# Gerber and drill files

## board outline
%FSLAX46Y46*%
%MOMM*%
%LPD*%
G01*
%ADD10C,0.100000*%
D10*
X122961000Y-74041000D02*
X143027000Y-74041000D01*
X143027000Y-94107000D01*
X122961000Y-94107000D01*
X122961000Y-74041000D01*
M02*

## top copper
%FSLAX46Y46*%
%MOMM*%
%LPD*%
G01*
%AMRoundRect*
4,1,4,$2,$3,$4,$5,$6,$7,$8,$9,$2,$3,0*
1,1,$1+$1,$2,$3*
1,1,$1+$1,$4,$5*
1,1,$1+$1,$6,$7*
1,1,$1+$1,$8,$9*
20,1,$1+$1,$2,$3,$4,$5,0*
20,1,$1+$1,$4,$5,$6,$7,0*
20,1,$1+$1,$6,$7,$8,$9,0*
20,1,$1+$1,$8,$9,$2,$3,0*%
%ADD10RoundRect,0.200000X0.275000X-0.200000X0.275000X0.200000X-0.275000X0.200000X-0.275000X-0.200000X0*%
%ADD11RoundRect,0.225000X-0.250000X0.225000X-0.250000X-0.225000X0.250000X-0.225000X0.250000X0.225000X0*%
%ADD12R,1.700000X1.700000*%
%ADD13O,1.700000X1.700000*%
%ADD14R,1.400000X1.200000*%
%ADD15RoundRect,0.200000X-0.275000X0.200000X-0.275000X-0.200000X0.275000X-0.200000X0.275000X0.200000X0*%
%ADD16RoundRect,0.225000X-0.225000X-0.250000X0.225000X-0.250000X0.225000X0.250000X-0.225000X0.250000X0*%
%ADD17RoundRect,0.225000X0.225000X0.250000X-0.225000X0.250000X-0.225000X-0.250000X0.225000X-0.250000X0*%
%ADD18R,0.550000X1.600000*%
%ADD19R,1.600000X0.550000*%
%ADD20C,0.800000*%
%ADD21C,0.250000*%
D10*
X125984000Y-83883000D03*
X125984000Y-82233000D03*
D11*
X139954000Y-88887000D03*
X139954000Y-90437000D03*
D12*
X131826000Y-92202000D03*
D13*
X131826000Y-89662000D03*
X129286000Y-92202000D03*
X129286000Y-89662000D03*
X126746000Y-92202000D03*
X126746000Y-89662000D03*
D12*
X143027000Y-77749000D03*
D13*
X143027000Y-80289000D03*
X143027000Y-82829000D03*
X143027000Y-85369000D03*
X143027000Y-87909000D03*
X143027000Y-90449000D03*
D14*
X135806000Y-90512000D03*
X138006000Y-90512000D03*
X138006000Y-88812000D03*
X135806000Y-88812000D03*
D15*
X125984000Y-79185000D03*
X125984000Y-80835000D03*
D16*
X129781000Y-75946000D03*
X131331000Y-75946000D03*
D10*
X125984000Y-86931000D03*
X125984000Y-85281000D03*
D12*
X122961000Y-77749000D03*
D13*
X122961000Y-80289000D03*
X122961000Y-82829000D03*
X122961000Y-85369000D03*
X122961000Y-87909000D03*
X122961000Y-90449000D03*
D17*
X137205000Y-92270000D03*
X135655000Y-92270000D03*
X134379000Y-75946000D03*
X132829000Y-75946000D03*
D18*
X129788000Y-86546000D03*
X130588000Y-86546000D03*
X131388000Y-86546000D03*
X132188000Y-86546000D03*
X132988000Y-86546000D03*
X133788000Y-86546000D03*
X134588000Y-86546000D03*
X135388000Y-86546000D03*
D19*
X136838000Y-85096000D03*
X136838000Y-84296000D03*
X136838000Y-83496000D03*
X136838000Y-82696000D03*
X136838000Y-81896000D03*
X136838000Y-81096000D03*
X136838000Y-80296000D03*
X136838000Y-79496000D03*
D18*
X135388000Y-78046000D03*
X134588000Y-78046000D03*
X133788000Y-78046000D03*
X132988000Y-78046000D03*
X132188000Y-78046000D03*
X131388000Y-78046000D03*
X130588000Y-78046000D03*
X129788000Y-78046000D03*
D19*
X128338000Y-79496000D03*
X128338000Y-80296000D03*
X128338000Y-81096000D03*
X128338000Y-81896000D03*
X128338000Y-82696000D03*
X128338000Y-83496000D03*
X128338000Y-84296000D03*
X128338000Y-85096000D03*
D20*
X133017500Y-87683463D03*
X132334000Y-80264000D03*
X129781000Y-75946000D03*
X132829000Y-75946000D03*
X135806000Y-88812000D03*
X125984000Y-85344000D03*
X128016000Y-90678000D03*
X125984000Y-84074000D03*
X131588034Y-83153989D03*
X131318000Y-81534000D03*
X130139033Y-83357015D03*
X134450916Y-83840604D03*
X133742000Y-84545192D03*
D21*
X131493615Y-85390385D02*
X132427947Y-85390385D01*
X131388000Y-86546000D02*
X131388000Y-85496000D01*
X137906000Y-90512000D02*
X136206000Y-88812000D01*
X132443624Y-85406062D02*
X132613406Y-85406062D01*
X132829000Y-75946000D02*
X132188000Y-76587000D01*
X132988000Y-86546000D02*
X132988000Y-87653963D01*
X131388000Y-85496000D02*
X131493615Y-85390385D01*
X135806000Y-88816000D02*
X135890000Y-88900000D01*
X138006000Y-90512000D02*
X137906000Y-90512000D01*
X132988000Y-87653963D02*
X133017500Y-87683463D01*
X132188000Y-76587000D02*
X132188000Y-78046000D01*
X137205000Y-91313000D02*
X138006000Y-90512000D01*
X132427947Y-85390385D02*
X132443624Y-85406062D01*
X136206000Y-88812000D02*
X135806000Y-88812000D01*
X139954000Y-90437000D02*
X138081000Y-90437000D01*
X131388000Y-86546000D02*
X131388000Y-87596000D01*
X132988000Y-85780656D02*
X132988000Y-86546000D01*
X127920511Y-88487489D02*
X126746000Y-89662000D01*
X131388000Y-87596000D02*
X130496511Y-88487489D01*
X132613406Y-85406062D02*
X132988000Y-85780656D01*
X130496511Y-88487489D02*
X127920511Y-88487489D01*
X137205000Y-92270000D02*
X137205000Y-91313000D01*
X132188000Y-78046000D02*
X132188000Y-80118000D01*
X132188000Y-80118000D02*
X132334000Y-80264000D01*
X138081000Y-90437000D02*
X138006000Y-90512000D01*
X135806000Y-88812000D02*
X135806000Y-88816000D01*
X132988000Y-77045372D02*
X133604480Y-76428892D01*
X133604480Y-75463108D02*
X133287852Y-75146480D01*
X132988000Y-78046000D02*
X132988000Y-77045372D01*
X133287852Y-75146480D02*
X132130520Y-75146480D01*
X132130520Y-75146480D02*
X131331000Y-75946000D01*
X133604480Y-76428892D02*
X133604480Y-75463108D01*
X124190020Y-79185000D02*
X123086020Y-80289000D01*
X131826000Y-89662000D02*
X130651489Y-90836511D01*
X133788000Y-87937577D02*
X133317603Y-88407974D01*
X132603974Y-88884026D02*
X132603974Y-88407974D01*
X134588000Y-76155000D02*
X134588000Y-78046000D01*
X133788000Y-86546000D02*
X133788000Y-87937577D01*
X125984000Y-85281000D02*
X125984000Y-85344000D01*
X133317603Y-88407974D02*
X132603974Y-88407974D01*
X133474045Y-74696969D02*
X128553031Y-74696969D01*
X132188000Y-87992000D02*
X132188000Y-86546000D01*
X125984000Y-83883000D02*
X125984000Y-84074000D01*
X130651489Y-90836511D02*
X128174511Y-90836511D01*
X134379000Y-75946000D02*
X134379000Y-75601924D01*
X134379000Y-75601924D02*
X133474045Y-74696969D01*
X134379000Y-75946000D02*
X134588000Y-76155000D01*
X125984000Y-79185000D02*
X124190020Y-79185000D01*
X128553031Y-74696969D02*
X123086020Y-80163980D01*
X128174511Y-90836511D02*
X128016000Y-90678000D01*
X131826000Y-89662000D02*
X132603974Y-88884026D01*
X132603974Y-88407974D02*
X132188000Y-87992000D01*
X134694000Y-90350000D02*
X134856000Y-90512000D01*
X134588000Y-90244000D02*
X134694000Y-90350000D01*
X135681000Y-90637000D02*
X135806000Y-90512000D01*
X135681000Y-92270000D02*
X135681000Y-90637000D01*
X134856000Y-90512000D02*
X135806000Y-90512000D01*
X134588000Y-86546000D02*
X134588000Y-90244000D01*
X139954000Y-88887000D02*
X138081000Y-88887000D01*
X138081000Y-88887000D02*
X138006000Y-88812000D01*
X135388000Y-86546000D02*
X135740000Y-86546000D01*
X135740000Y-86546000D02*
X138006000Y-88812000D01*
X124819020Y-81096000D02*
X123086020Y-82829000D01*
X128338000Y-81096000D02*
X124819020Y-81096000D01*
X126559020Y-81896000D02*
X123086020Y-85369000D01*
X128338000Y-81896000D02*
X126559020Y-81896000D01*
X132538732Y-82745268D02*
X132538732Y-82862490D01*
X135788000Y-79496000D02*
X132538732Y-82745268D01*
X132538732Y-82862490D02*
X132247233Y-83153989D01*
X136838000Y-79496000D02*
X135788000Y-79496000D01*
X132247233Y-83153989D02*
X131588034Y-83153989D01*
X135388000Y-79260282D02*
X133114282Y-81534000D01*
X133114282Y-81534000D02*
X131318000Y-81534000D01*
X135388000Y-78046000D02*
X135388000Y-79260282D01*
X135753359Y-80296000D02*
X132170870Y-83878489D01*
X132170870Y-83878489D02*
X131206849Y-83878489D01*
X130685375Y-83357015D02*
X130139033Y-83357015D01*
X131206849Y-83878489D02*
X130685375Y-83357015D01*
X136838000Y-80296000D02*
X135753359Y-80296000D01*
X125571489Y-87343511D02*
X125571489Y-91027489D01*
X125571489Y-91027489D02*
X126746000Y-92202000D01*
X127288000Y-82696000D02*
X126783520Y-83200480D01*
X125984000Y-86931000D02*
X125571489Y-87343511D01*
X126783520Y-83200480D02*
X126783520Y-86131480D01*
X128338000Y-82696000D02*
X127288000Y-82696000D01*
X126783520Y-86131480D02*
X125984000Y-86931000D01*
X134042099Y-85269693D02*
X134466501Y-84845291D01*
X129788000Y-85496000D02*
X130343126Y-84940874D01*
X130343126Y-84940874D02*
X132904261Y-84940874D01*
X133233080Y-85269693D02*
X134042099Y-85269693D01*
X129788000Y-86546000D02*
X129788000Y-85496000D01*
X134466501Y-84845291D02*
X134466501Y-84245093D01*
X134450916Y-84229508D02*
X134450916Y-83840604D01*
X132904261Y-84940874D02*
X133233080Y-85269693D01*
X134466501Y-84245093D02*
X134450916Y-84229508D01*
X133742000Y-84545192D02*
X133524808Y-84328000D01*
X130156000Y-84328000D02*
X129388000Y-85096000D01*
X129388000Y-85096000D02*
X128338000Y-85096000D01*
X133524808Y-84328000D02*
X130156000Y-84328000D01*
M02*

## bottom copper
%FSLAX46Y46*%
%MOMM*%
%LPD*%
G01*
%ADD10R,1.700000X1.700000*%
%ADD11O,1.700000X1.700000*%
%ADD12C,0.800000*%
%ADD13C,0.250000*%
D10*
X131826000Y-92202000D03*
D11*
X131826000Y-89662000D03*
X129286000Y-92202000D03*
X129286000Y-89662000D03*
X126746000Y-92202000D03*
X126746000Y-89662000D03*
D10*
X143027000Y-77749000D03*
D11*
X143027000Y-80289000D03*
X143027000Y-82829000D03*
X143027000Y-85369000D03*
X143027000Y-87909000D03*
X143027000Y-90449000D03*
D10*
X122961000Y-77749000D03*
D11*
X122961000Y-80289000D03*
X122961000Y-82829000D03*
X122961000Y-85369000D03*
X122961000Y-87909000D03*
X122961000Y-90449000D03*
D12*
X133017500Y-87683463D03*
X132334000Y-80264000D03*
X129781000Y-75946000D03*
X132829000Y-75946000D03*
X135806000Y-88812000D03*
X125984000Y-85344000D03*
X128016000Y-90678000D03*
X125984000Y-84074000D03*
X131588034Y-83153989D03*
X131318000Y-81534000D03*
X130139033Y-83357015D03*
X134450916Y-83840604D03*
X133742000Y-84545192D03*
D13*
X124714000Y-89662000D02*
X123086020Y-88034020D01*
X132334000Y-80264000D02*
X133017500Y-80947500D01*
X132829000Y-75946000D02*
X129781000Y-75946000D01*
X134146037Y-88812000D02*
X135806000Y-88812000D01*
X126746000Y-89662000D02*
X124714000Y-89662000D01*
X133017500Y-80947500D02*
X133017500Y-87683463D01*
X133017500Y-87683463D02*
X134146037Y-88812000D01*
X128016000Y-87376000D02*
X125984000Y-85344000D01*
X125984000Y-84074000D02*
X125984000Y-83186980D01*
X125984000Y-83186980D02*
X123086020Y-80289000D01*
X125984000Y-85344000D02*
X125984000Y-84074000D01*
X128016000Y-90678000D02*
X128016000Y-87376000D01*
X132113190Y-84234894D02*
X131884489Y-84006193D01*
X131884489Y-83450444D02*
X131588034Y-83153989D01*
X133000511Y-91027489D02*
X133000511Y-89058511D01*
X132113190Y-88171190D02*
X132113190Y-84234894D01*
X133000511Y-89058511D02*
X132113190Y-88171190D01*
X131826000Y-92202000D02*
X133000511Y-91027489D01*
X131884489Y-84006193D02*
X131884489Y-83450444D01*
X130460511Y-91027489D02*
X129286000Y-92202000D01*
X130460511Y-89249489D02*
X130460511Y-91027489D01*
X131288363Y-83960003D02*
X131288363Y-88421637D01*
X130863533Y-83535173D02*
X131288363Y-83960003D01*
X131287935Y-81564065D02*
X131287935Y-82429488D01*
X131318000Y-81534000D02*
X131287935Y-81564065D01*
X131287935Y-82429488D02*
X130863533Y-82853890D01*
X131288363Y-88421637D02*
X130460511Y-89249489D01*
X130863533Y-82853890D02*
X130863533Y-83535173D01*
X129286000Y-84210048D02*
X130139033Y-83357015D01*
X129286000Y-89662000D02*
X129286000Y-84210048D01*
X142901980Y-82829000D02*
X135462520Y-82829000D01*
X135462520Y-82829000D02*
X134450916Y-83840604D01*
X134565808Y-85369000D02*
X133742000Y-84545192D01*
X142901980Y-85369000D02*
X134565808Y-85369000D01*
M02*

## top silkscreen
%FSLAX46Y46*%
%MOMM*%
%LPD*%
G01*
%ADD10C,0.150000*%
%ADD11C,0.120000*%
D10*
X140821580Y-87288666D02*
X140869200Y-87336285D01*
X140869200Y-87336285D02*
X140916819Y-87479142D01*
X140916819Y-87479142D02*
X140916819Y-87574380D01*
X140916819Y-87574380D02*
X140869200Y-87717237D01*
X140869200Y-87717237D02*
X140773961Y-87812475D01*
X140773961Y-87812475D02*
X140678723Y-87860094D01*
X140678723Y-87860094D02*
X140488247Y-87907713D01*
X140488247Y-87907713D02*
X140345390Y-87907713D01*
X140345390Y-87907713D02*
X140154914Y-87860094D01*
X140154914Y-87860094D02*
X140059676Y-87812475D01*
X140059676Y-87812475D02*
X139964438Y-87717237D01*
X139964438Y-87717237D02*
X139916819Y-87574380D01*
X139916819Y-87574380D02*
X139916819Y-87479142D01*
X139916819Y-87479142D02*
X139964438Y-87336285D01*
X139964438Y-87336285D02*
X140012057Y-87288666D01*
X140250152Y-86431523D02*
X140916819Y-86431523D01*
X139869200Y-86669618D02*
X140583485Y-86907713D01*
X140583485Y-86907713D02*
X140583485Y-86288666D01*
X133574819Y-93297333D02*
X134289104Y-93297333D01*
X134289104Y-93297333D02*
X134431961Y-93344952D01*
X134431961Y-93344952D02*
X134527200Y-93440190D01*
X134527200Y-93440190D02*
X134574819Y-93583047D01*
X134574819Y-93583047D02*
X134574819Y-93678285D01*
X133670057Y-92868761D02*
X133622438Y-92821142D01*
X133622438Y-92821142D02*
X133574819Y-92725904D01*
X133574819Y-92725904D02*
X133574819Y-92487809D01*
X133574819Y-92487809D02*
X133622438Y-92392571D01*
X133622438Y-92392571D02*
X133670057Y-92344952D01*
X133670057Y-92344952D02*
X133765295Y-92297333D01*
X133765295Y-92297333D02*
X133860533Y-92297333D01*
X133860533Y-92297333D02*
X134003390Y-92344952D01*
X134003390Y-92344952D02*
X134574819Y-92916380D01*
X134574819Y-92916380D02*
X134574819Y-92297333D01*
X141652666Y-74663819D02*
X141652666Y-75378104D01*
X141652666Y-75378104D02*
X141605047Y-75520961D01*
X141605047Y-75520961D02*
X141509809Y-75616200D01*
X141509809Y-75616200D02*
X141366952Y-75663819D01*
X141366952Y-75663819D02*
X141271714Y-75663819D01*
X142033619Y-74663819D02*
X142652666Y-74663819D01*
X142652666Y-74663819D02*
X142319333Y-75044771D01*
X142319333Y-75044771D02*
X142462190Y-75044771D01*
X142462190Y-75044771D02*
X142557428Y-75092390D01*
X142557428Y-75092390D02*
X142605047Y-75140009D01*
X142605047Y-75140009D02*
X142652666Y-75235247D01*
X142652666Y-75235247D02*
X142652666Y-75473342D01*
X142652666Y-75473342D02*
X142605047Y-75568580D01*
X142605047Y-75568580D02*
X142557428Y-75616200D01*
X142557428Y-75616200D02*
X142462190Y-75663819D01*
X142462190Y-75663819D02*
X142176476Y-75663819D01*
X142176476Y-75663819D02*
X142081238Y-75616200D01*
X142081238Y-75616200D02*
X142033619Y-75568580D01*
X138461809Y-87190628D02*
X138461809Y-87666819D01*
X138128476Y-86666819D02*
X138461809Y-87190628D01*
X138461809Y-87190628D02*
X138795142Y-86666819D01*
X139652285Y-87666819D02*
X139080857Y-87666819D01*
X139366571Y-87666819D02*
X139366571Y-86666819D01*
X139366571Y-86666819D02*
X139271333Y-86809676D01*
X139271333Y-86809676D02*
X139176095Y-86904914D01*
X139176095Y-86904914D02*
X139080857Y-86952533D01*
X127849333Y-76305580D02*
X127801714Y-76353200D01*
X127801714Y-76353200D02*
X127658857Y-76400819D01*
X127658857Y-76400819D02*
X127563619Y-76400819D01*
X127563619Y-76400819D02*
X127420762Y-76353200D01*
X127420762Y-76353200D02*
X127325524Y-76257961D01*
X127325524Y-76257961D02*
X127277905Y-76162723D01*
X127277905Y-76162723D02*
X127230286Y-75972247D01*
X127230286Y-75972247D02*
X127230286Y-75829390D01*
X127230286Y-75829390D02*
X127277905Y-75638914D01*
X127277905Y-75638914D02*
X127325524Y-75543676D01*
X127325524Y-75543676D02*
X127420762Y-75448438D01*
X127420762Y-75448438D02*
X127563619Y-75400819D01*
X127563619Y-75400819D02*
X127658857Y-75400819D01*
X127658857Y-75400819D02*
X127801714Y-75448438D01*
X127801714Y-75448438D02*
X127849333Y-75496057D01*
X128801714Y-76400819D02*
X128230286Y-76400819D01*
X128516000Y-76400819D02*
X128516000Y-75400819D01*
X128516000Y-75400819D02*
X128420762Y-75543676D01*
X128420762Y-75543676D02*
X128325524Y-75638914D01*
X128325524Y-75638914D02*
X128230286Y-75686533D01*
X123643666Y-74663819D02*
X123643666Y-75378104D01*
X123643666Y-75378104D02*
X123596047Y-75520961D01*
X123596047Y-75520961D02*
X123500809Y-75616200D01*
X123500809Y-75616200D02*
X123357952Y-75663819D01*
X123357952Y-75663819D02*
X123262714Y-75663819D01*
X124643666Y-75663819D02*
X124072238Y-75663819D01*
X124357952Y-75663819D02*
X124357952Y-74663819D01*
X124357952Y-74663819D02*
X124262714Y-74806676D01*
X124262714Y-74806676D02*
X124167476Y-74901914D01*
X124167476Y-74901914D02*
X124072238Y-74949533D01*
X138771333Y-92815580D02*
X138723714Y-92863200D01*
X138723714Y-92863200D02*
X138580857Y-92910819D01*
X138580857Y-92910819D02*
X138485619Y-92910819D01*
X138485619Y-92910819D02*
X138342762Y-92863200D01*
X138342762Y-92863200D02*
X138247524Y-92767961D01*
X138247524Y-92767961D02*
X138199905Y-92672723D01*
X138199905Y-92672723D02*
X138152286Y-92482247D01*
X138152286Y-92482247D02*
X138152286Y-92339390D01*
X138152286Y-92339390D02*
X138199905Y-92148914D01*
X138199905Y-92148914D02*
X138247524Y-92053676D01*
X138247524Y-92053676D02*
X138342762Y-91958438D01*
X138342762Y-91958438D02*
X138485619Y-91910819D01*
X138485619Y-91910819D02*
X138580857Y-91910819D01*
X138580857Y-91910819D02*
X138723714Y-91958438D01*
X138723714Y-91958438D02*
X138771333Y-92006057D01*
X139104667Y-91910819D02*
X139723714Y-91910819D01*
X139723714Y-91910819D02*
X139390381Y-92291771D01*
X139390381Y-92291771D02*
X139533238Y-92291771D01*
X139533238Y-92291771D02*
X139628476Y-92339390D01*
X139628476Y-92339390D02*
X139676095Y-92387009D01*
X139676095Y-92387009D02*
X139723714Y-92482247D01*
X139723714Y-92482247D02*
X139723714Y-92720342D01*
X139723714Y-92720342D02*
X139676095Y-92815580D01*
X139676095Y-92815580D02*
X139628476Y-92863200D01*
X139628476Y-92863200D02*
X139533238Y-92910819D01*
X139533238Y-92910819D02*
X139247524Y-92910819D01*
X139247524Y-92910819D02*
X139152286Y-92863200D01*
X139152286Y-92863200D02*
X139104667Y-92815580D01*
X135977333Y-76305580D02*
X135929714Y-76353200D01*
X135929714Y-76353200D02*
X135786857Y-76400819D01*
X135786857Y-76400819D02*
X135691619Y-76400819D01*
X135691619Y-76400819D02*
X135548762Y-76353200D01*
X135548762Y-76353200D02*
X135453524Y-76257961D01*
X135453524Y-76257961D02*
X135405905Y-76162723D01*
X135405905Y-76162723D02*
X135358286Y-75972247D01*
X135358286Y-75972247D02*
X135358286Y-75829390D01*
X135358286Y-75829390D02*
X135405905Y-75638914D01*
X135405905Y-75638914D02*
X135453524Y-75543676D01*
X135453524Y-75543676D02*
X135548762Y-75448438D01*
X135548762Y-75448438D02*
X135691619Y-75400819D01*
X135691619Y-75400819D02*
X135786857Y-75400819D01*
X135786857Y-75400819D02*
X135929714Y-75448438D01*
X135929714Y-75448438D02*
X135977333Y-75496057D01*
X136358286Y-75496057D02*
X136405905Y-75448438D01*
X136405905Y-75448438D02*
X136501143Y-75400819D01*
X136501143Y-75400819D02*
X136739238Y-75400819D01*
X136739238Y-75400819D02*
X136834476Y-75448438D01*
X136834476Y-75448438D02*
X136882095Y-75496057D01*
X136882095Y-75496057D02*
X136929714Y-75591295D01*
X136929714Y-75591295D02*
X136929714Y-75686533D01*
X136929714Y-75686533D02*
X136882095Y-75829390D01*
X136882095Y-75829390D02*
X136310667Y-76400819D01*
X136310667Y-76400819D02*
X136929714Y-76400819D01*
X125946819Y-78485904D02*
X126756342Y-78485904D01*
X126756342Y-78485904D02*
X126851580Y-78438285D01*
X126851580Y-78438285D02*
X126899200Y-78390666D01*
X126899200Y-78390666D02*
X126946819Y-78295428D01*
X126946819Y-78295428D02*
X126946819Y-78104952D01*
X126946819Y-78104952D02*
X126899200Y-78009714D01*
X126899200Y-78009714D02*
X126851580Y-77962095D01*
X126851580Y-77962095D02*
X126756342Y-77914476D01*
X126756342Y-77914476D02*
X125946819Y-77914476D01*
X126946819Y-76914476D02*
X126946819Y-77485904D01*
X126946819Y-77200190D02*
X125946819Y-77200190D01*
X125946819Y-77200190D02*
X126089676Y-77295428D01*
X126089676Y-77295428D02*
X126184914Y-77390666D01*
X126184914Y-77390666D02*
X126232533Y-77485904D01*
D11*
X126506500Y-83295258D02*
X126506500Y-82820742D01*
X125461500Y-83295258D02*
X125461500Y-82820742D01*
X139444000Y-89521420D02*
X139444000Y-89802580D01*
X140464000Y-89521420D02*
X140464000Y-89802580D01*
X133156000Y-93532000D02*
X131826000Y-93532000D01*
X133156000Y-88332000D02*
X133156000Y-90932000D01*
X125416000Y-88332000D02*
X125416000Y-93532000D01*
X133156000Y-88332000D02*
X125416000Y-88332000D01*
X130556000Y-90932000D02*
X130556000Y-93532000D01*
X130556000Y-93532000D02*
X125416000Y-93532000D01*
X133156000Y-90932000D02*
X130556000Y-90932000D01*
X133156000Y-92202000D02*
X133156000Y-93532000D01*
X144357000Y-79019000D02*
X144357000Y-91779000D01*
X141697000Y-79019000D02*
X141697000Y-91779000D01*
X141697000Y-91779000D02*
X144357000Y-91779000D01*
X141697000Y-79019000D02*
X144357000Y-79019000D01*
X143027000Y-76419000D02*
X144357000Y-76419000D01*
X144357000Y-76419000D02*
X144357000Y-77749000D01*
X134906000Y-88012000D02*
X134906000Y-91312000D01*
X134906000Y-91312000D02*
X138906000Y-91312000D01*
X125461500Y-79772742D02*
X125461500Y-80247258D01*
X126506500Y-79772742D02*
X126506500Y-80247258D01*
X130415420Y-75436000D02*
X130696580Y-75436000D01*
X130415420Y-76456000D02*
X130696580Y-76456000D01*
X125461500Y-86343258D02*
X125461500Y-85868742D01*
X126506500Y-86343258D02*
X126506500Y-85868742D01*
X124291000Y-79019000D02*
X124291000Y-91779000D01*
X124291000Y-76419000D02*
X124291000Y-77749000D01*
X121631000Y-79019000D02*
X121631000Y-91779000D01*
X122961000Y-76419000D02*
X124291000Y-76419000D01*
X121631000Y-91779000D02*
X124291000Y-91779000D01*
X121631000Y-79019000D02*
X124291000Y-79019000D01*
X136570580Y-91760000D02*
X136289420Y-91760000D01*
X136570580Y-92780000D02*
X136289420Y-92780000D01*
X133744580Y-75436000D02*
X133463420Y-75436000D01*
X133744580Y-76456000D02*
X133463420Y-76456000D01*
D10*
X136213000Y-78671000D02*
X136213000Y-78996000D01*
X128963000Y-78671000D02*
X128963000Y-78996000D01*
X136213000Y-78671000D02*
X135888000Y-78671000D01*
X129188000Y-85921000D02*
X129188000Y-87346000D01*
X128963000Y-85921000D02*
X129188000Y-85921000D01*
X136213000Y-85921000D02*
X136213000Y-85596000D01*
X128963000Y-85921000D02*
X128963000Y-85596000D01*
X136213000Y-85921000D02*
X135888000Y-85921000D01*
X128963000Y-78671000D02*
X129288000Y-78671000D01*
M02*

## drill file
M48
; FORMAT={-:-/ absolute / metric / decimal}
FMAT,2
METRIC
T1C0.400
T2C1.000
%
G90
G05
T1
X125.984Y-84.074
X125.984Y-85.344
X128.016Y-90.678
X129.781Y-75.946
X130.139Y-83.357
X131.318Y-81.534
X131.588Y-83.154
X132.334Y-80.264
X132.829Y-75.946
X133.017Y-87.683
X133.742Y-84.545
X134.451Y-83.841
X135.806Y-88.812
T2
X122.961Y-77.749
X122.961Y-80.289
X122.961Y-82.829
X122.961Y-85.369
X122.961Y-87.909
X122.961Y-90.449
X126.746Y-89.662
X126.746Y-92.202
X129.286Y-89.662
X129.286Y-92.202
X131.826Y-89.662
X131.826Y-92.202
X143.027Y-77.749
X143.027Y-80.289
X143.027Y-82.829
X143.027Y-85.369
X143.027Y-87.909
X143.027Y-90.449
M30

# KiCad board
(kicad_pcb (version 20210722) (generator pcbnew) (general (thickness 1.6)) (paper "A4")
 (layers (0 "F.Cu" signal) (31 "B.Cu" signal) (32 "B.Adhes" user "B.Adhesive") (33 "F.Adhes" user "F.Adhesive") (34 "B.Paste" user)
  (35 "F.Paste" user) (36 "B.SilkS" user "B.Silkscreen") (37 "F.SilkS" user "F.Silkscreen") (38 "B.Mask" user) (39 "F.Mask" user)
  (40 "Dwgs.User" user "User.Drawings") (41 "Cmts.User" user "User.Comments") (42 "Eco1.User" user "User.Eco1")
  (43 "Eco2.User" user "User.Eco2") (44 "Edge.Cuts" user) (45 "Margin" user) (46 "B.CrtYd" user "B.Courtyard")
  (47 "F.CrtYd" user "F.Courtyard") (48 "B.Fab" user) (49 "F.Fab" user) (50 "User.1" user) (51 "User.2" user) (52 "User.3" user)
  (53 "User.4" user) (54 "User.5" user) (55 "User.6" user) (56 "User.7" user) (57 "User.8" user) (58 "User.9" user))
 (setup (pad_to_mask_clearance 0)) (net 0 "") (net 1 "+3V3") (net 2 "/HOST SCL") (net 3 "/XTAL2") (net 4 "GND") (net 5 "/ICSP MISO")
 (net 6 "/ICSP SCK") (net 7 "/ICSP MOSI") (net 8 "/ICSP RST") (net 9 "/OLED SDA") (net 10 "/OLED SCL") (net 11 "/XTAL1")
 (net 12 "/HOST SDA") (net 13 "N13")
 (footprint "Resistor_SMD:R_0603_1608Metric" (layer "F.Cu") (at 125.984 83.058 90)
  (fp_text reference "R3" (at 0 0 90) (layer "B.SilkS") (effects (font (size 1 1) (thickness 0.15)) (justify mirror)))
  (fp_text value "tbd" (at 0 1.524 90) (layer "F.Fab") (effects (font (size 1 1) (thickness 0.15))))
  (fp_line (start -0.237258 0.5225) (end 0.237258 0.5225) (layer "F.SilkS") (width 0.12))
  (fp_line (start -0.237258 -0.5225) (end 0.237258 -0.5225) (layer "F.SilkS") (width 0.12))
  (pad "1" smd roundrect locked (at -0.825 0 90) (size 0.8 0.95) (layers "F.Cu" "F.Paste" "F.Mask") (roundrect_rratio 0.25) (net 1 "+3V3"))
  (pad "2" smd roundrect locked (at 0.825 0 90) (size 0.8 0.95) (layers "F.Cu" "F.Paste" "F.Mask") (roundrect_rratio 0.25)
   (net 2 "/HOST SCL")))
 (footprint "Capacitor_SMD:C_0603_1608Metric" (layer "F.Cu") (at 139.954 89.662 -90)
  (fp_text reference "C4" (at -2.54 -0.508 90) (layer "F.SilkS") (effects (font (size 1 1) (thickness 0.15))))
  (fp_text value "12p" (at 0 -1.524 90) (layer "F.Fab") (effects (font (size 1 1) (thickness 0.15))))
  (fp_line (start -0.14058 0.51) (end 0.14058 0.51) (layer "F.SilkS") (width 0.12))
  (fp_line (start -0.14058 -0.51) (end 0.14058 -0.51) (layer "F.SilkS") (width 0.12))
  (pad "1" smd roundrect locked (at -0.775 0 270) (size 0.9 0.95) (layers "F.Cu" "F.Paste" "F.Mask") (roundrect_rratio 0.25)
   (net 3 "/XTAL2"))
  (pad "2" smd roundrect locked (at 0.775 0 270) (size 0.9 0.95) (layers "F.Cu" "F.Paste" "F.Mask") (roundrect_rratio 0.25) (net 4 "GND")))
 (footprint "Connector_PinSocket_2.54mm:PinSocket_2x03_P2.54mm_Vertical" (layer "F.Cu") (at 131.826 92.202 -90)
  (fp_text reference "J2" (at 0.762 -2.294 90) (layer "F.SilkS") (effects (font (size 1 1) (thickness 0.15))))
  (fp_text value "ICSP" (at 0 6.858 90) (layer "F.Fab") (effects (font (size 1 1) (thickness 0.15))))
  (fp_line (start 1.33 -1.33) (end 1.33 0) (layer "F.SilkS") (width 0.12))
  (fp_line (start -3.87 -1.33) (end -1.27 -1.33) (layer "F.SilkS") (width 0.12))
  (fp_line (start -3.87 6.41) (end 1.33 6.41) (layer "F.SilkS") (width 0.12))
  (fp_line (start -3.87 -1.33) (end -3.87 6.41) (layer "F.SilkS") (width 0.12))
  (fp_line (start -1.27 1.27) (end 1.33 1.27) (layer "F.SilkS") (width 0.12))
  (fp_line (start 1.33 1.27) (end 1.33 6.41) (layer "F.SilkS") (width 0.12))
  (fp_line (start -1.27 -1.33) (end -1.27 1.27) (layer "F.SilkS") (width 0.12))
  (fp_line (start 0 -1.33) (end 1.33 -1.33) (layer "F.SilkS") (width 0.12))
  (pad "1" thru_hole rect locked (at 0 0 270) (size 1.7 1.7) (drill 1) (layers *.Cu *.Mask) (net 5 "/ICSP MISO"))
  (pad "2" thru_hole oval locked (at -2.54 0 270) (size 1.7 1.7) (drill 1) (layers *.Cu *.Mask) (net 1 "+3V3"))
  (pad "3" thru_hole oval locked (at 0 2.54 270) (size 1.7 1.7) (drill 1) (layers *.Cu *.Mask) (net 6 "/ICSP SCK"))
  (pad "4" thru_hole oval locked (at -2.54 2.54 270) (size 1.7 1.7) (drill 1) (layers *.Cu *.Mask) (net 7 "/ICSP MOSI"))
  (pad "5" thru_hole oval locked (at 0 5.08 270) (size 1.7 1.7) (drill 1) (layers *.Cu *.Mask) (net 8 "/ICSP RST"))
  (pad "6" thru_hole oval locked (at -2.54 5.08 270) (size 1.7 1.7) (drill 1) (layers *.Cu *.Mask) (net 4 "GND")))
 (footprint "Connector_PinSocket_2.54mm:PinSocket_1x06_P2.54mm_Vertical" (layer "F.Cu") (at 143.027 77.749)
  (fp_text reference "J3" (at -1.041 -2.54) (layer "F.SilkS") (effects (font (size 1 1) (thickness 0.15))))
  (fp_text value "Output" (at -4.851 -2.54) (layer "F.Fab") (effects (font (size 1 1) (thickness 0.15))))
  (fp_line (start 1.33 1.27) (end 1.33 14.03) (layer "F.SilkS") (width 0.12))
  (fp_line (start -1.33 1.27) (end -1.33 14.03) (layer "F.SilkS") (width 0.12))
  (fp_line (start -1.33 14.03) (end 1.33 14.03) (layer "F.SilkS") (width 0.12))
  (fp_line (start -1.33 1.27) (end 1.33 1.27) (layer "F.SilkS") (width 0.12))
  (fp_line (start 0 -1.33) (end 1.33 -1.33) (layer "F.SilkS") (width 0.12))
  (fp_line (start 1.33 -1.33) (end 1.33 0) (layer "F.SilkS") (width 0.12))
  (pad "1" thru_hole rect locked (at 0 0) (size 1.7 1.7) (drill 1) (layers *.Cu *.Mask))
  (pad "2" thru_hole oval locked (at 0 2.54) (size 1.7 1.7) (drill 1) (layers *.Cu *.Mask))
  (pad "3" thru_hole oval locked (at 0 5.08) (size 1.7 1.7) (drill 1) (layers *.Cu *.Mask) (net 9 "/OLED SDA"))
  (pad "4" thru_hole oval locked (at 0 7.62) (size 1.7 1.7) (drill 1) (layers *.Cu *.Mask) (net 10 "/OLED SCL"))
  (pad "5" thru_hole oval locked (at 0 10.16) (size 1.7 1.7) (drill 1) (layers *.Cu *.Mask))
  (pad "6" thru_hole oval locked (at 0 12.7) (size 1.7 1.7) (drill 1) (layers *.Cu *.Mask)))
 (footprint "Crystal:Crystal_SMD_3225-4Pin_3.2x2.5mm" (layer "F.Cu") (at 136.906 89.662)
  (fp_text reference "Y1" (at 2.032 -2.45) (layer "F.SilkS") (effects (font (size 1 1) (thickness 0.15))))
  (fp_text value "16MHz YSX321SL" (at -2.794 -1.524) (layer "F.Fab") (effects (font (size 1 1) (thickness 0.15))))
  (fp_line (start -2 -1.65) (end -2 1.65) (layer "F.SilkS") (width 0.12))
  (fp_line (start -2 1.65) (end 2 1.65) (layer "F.SilkS") (width 0.12))
  (pad "1" smd rect locked (at -1.1 0.85) (size 1.4 1.2) (layers "F.Cu" "F.Paste" "F.Mask") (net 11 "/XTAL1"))
  (pad "2" smd rect locked (at 1.1 0.85) (size 1.4 1.2) (layers "F.Cu" "F.Paste" "F.Mask") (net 4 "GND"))
  (pad "3" smd rect locked (at 1.1 -0.85) (size 1.4 1.2) (layers "F.Cu" "F.Paste" "F.Mask") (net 3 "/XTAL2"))
  (pad "4" smd rect locked (at -1.1 -0.85) (size 1.4 1.2) (layers "F.Cu" "F.Paste" "F.Mask") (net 4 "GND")))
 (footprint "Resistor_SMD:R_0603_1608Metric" (layer "F.Cu") (at 125.984 80.01 -90)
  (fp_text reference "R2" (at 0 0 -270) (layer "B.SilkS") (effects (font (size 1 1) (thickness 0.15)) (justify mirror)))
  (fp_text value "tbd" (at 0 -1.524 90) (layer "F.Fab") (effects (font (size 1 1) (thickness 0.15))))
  (fp_line (start -0.237258 0.5225) (end 0.237258 0.5225) (layer "F.SilkS") (width 0.12))
  (fp_line (start -0.237258 -0.5225) (end 0.237258 -0.5225) (layer "F.SilkS") (width 0.12))
  (pad "1" smd roundrect locked (at -0.825 0 270) (size 0.8 0.95) (layers "F.Cu" "F.Paste" "F.Mask") (roundrect_rratio 0.25) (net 1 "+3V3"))
  (pad "2" smd roundrect locked (at 0.825 0 270) (size 0.8 0.95) (layers "F.Cu" "F.Paste" "F.Mask") (roundrect_rratio 0.25)
   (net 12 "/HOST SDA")))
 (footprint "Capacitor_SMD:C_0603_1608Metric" (layer "F.Cu") (at 130.556 75.946)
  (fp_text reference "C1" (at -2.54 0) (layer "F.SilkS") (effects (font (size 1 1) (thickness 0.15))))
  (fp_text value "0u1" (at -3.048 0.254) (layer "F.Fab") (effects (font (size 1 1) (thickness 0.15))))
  (fp_line (start -0.14058 -0.51) (end 0.14058 -0.51) (layer "F.SilkS") (width 0.12))
  (fp_line (start -0.14058 0.51) (end 0.14058 0.51) (layer "F.SilkS") (width 0.12))
  (pad "1" smd roundrect locked (at -0.775 0) (size 0.9 0.95) (layers "F.Cu" "F.Paste" "F.Mask") (roundrect_rratio 0.25) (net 4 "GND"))
  (pad "2" smd roundrect locked (at 0.775 0) (size 0.9 0.95) (layers "F.Cu" "F.Paste" "F.Mask") (roundrect_rratio 0.25) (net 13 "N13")))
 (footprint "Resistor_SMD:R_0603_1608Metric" (layer "F.Cu") (at 125.984 86.106 90)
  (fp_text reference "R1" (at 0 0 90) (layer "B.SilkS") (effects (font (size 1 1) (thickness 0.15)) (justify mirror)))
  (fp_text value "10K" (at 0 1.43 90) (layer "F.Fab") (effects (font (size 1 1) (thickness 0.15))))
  (fp_line (start -0.237258 -0.5225) (end 0.237258 -0.5225) (layer "F.SilkS") (width 0.12))
  (fp_line (start -0.237258 0.5225) (end 0.237258 0.5225) (layer "F.SilkS") (width 0.12))
  (pad "1" smd roundrect locked (at -0.825 0 90) (size 0.8 0.95) (layers "F.Cu" "F.Paste" "F.Mask") (roundrect_rratio 0.25)
   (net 8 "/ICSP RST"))
  (pad "2" smd roundrect locked (at 0.825 0 90) (size 0.8 0.95) (layers "F.Cu" "F.Paste" "F.Mask") (roundrect_rratio 0.25) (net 1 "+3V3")))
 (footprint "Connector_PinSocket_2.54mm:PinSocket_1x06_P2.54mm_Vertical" (layer "F.Cu") (at 122.961 77.749)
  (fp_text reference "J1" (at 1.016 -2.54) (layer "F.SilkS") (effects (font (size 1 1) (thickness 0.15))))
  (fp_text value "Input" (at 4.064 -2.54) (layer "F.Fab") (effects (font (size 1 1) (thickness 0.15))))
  (fp_line (start 1.33 1.27) (end 1.33 14.03) (layer "F.SilkS") (width 0.12))
  (fp_line (start 1.33 -1.33) (end 1.33 0) (layer "F.SilkS") (width 0.12))
  (fp_line (start -1.33 1.27) (end -1.33 14.03) (layer "F.SilkS") (width 0.12))
  (fp_line (start 0 -1.33) (end 1.33 -1.33) (layer "F.SilkS") (width 0.12))
  (fp_line (start -1.33 14.03) (end 1.33 14.03) (layer "F.SilkS") (width 0.12))
  (fp_line (start -1.33 1.27) (end 1.33 1.27) (layer "F.SilkS") (width 0.12))
  (pad "1" thru_hole rect locked (at 0 0) (size 1.7 1.7) (drill 1) (layers *.Cu *.Mask))
  (pad "2" thru_hole oval locked (at 0 2.54) (size 1.7 1.7) (drill 1) (layers *.Cu *.Mask) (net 1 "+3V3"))
  (pad "3" thru_hole oval locked (at 0 5.08) (size 1.7 1.7) (drill 1) (layers *.Cu *.Mask) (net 12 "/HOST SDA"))
  (pad "4" thru_hole oval locked (at 0 7.62) (size 1.7 1.7) (drill 1) (layers *.Cu *.Mask) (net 2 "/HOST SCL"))
  (pad "5" thru_hole oval locked (at 0 10.16) (size 1.7 1.7) (drill 1) (layers *.Cu *.Mask) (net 4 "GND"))
  (pad "6" thru_hole oval locked (at 0 12.7) (size 1.7 1.7) (drill 1) (layers *.Cu *.Mask)))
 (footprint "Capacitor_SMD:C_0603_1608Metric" (layer "F.Cu") (at 136.43 92.27 180)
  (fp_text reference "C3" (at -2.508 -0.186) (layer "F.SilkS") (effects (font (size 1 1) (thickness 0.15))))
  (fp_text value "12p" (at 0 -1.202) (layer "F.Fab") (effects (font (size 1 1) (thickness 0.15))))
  (fp_line (start -0.14058 0.51) (end 0.14058 0.51) (layer "F.SilkS") (width 0.12))
  (fp_line (start -0.14058 -0.51) (end 0.14058 -0.51) (layer "F.SilkS") (width 0.12))
  (pad "1" smd roundrect locked (at -0.775 0 180) (size 0.9 0.95) (layers "F.Cu" "F.Paste" "F.Mask") (roundrect_rratio 0.25) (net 4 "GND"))
  (pad "2" smd roundrect locked (at 0.775 0 180) (size 0.9 0.95) (layers "F.Cu" "F.Paste" "F.Mask") (roundrect_rratio 0.25)
   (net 11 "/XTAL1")))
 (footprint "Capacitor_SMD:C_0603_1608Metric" (layer "F.Cu") (at 133.604 75.946 180)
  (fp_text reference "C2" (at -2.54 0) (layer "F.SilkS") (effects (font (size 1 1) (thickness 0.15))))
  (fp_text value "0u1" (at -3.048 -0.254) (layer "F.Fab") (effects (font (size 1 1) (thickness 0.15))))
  (fp_line (start -0.14058 0.51) (end 0.14058 0.51) (layer "F.SilkS") (width 0.12))
  (fp_line (start -0.14058 -0.51) (end 0.14058 -0.51) (layer "F.SilkS") (width 0.12))
  (pad "1" smd roundrect locked (at -0.775 0 180) (size 0.9 0.95) (layers "F.Cu" "F.Paste" "F.Mask") (roundrect_rratio 0.25) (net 1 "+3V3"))
  (pad "2" smd roundrect locked (at 0.775 0 180) (size 0.9 0.95) (layers "F.Cu" "F.Paste" "F.Mask") (roundrect_rratio 0.25) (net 4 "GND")))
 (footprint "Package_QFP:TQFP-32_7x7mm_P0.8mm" (layer "F.Cu") (at 132.588 82.296 90)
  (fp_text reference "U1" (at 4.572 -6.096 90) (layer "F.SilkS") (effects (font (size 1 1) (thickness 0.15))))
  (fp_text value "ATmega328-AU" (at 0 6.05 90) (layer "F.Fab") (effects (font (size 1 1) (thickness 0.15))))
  (fp_line (start 3.625 3.625) (end 3.3 3.625) (layer "F.SilkS") (width 0.15))
  (fp_line (start 3.625 -3.625) (end 3.3 -3.625) (layer "F.SilkS") (width 0.15))
  (fp_line (start 3.625 3.625) (end 3.625 3.3) (layer "F.SilkS") (width 0.15))
  (fp_line (start -3.625 -3.4) (end -5.05 -3.4) (layer "F.SilkS") (width 0.15))
  (fp_line (start -3.625 -3.625) (end -3.625 -3.4) (layer "F.SilkS") (width 0.15))
  (fp_line (start -3.625 3.625) (end -3.3 3.625) (layer "F.SilkS") (width 0.15))
  (fp_line (start -3.625 -3.625) (end -3.3 -3.625) (layer "F.SilkS") (width 0.15))
  (fp_line (start -3.625 3.625) (end -3.625 3.3) (layer "F.SilkS") (width 0.15))
  (fp_line (start 3.625 -3.625) (end 3.625 -3.3) (layer "F.SilkS") (width 0.15))
  (pad "1" smd rect locked (at -4.25 -2.8 90) (size 1.6 0.55) (layers "F.Cu" "F.Paste" "F.Mask") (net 9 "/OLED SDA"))
  (pad "2" smd rect locked (at -4.25 -2 90) (size 1.6 0.55) (layers "F.Cu" "F.Paste" "F.Mask"))
  (pad "3" smd rect locked (at -4.25 -1.2 90) (size 1.6 0.55) (layers "F.Cu" "F.Paste" "F.Mask") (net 4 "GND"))
  (pad "4" smd rect locked (at -4.25 -0.4 90) (size 1.6 0.55) (layers "F.Cu" "F.Paste" "F.Mask") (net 1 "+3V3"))
  (pad "5" smd rect locked (at -4.25 0.4 90) (size 1.6 0.55) (layers "F.Cu" "F.Paste" "F.Mask") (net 4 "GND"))
  (pad "6" smd rect locked (at -4.25 1.2 90) (size 1.6 0.55) (layers "F.Cu" "F.Paste" "F.Mask") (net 1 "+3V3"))
  (pad "7" smd rect locked (at -4.25 2 90) (size 1.6 0.55) (layers "F.Cu" "F.Paste" "F.Mask") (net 11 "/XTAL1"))
  (pad "8" smd rect locked (at -4.25 2.8 90) (size 1.6 0.55) (layers "F.Cu" "F.Paste" "F.Mask") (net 3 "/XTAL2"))
  (pad "9" smd rect locked (at -2.8 4.25 180) (size 1.6 0.55) (layers "F.Cu" "F.Paste" "F.Mask"))
  (pad "10" smd rect locked (at -2 4.25 180) (size 1.6 0.55) (layers "F.Cu" "F.Paste" "F.Mask"))
  (pad "11" smd rect locked (at -1.2 4.25 180) (size 1.6 0.55) (layers "F.Cu" "F.Paste" "F.Mask"))
  (pad "12" smd rect locked (at -0.4 4.25 180) (size 1.6 0.55) (layers "F.Cu" "F.Paste" "F.Mask"))
  (pad "13" smd rect locked (at 0.4 4.25 180) (size 1.6 0.55) (layers "F.Cu" "F.Paste" "F.Mask"))
  (pad "14" smd rect locked (at 1.2 4.25 180) (size 1.6 0.55) (layers "F.Cu" "F.Paste" "F.Mask"))
  (pad "15" smd rect locked (at 2 4.25 180) (size 1.6 0.55) (layers "F.Cu" "F.Paste" "F.Mask") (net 7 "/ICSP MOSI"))
  (pad "16" smd rect locked (at 2.8 4.25 180) (size 1.6 0.55) (layers "F.Cu" "F.Paste" "F.Mask") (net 5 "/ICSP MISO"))
  (pad "17" smd rect locked (at 4.25 2.8 90) (size 1.6 0.55) (layers "F.Cu" "F.Paste" "F.Mask") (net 6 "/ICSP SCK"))
  (pad "18" smd rect locked (at 4.25 2 90) (size 1.6 0.55) (layers "F.Cu" "F.Paste" "F.Mask") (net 1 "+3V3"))
  (pad "19" smd rect locked (at 4.25 1.2 90) (size 1.6 0.55) (layers "F.Cu" "F.Paste" "F.Mask"))
  (pad "20" smd rect locked (at 4.25 0.4 90) (size 1.6 0.55) (layers "F.Cu" "F.Paste" "F.Mask") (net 13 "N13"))
  (pad "21" smd rect locked (at 4.25 -0.4 90) (size 1.6 0.55) (layers "F.Cu" "F.Paste" "F.Mask") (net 4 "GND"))
  (pad "22" smd rect locked (at 4.25 -1.2 90) (size 1.6 0.55) (layers "F.Cu" "F.Paste" "F.Mask"))
  (pad "23" smd rect locked (at 4.25 -2 90) (size 1.6 0.55) (layers "F.Cu" "F.Paste" "F.Mask"))
  (pad "24" smd rect locked (at 4.25 -2.8 90) (size 1.6 0.55) (layers "F.Cu" "F.Paste" "F.Mask"))
  (pad "25" smd rect locked (at 2.8 -4.25 180) (size 1.6 0.55) (layers "F.Cu" "F.Paste" "F.Mask"))
  (pad "26" smd rect locked (at 2 -4.25 180) (size 1.6 0.55) (layers "F.Cu" "F.Paste" "F.Mask"))
  (pad "27" smd rect locked (at 1.2 -4.25 180) (size 1.6 0.55) (layers "F.Cu" "F.Paste" "F.Mask") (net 12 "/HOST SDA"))
  (pad "28" smd rect locked (at 0.4 -4.25 180) (size 1.6 0.55) (layers "F.Cu" "F.Paste" "F.Mask") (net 2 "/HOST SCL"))
  (pad "29" smd rect locked (at -0.4 -4.25 180) (size 1.6 0.55) (layers "F.Cu" "F.Paste" "F.Mask") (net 8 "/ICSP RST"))
  (pad "30" smd rect locked (at -1.2 -4.25 180) (size 1.6 0.55) (layers "F.Cu" "F.Paste" "F.Mask"))
  (pad "31" smd rect locked (at -2 -4.25 180) (size 1.6 0.55) (layers "F.Cu" "F.Paste" "F.Mask"))
  (pad "32" smd rect locked (at -2.8 -4.25 180) (size 1.6 0.55) (layers "F.Cu" "F.Paste" "F.Mask") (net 10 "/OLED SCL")))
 (gr_rect (start 143.027 94.107) (end 122.961 74.041) (layer "Edge.Cuts") (width 0.1) (fill none))
 (segment (start 131.493615 85.390385) (end 132.427947 85.390385) (width 0.25) (layer "F.Cu") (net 4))
 (segment (start 131.388 86.546) (end 131.388 85.496) (width 0.25) (layer "F.Cu") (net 4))
 (segment (start 137.906 90.512) (end 136.206 88.812) (width 0.25) (layer "F.Cu") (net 4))
 (segment (start 132.443624 85.406062) (end 132.613406 85.406062) (width 0.25) (layer "F.Cu") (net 4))
 (segment (start 132.829 75.946) (end 132.188 76.587) (width 0.25) (layer "F.Cu") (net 4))
 (segment (start 132.988 86.546) (end 132.988 87.653963) (width 0.25) (layer "F.Cu") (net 4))
 (segment (start 131.388 85.496) (end 131.493615 85.390385) (width 0.25) (layer "F.Cu") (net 4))
 (segment (start 135.806 88.816) (end 135.89 88.9) (width 0.25) (layer "F.Cu") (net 4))
 (segment (start 138.006 90.512) (end 137.906 90.512) (width 0.25) (layer "F.Cu") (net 4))
 (segment (start 132.988 87.653963) (end 133.0175 87.683463) (width 0.25) (layer "F.Cu") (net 4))
 (segment (start 132.188 76.587) (end 132.188 78.046) (width 0.25) (layer "F.Cu") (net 4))
 (segment (start 137.205 91.313) (end 138.006 90.512) (width 0.25) (layer "F.Cu") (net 4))
 (segment (start 132.427947 85.390385) (end 132.443624 85.406062) (width 0.25) (layer "F.Cu") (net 4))
 (segment (start 136.206 88.812) (end 135.806 88.812) (width 0.25) (layer "F.Cu") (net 4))
 (segment (start 139.954 90.437) (end 138.081 90.437) (width 0.25) (layer "F.Cu") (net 4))
 (segment (start 131.388 86.546) (end 131.388 87.596) (width 0.25) (layer "F.Cu") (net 4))
 (segment (start 132.988 85.780656) (end 132.988 86.546) (width 0.25) (layer "F.Cu") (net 4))
 (segment (start 127.920511 88.487489) (end 126.746 89.662) (width 0.25) (layer "F.Cu") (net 4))
 (segment (start 131.388 87.596) (end 130.496511 88.487489) (width 0.25) (layer "F.Cu") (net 4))
 (segment (start 132.613406 85.406062) (end 132.988 85.780656) (width 0.25) (layer "F.Cu") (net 4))
 (segment (start 130.496511 88.487489) (end 127.920511 88.487489) (width 0.25) (layer "F.Cu") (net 4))
 (segment (start 137.205 92.27) (end 137.205 91.313) (width 0.25) (layer "F.Cu") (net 4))
 (segment (start 132.188 78.046) (end 132.188 80.118) (width 0.25) (layer "F.Cu") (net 4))
 (segment (start 132.188 80.118) (end 132.334 80.264) (width 0.25) (layer "F.Cu") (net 4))
 (segment (start 138.081 90.437) (end 138.006 90.512) (width 0.25) (layer "F.Cu") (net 4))
 (segment (start 135.806 88.812) (end 135.806 88.816) (width 0.25) (layer "F.Cu") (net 4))
 (via (at 133.0175 87.683463) (size 0.8) (drill 0.4) (layers "F.Cu" "B.Cu") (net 4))
 (via (at 132.334 80.264) (size 0.8) (drill 0.4) (layers "F.Cu" "B.Cu") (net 4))
 (via (at 129.781 75.946) (size 0.8) (drill 0.4) (layers "F.Cu" "B.Cu") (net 4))
 (via (at 132.829 75.946) (size 0.8) (drill 0.4) (layers "F.Cu" "B.Cu") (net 4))
 (via (at 135.806 88.812) (size 0.8) (drill 0.4) (layers "F.Cu" "B.Cu") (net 4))
 (segment (start 124.714 89.662) (end 123.08602 88.03402) (width 0.25) (layer "B.Cu") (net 4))
 (segment (start 132.334 80.264) (end 133.0175 80.9475) (width 0.25) (layer "B.Cu") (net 4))
 (segment (start 132.829 75.946) (end 129.781 75.946) (width 0.25) (layer "B.Cu") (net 4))
 (segment (start 134.146037 88.812) (end 135.806 88.812) (width 0.25) (layer "B.Cu") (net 4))
 (segment (start 126.746 89.662) (end 124.714 89.662) (width 0.25) (layer "B.Cu") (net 4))
 (segment (start 133.0175 80.9475) (end 133.0175 87.683463) (width 0.25) (layer "B.Cu") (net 4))
 (segment (start 133.0175 87.683463) (end 134.146037 88.812) (width 0.25) (layer "B.Cu") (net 4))
 (segment (start 132.988 77.045372) (end 133.60448 76.428892) (width 0.25) (layer "F.Cu") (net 13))
 (segment (start 133.60448 75.463108) (end 133.287852 75.14648) (width 0.25) (layer "F.Cu") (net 13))
 (segment (start 132.988 78.046) (end 132.988 77.045372) (width 0.25) (layer "F.Cu") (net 13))
 (segment (start 133.287852 75.14648) (end 132.13052 75.14648) (width 0.25) (layer "F.Cu") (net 13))
 (segment (start 132.13052 75.14648) (end 131.331 75.946) (width 0.25) (layer "F.Cu") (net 13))
 (segment (start 133.60448 76.428892) (end 133.60448 75.463108) (width 0.25) (layer "F.Cu") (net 13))
 (segment (start 124.19002 79.185) (end 123.08602 80.289) (width 0.25) (layer "F.Cu") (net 1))
 (segment (start 131.826 89.662) (end 130.651489 90.836511) (width 0.25) (layer "F.Cu") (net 1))
 (segment (start 133.788 87.937577) (end 133.317603 88.407974) (width 0.25) (layer "F.Cu") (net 1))
 (segment (start 132.603974 88.884026) (end 132.603974 88.407974) (width 0.25) (layer "F.Cu") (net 1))
 (segment (start 134.588 76.155) (end 134.588 78.046) (width 0.25) (layer "F.Cu") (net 1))
 (segment (start 133.788 86.546) (end 133.788 87.937577) (width 0.25) (layer "F.Cu") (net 1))
 (segment (start 125.984 85.281) (end 125.984 85.344) (width 0.25) (layer "F.Cu") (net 1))
 (segment (start 133.317603 88.407974) (end 132.603974 88.407974) (width 0.25) (layer "F.Cu") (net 1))
 (segment (start 133.474045 74.696969) (end 128.553031 74.696969) (width 0.25) (layer "F.Cu") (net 1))
 (segment (start 132.188 87.992) (end 132.188 86.546) (width 0.25) (layer "F.Cu") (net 1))
 (segment (start 125.984 83.883) (end 125.984 84.074) (width 0.25) (layer "F.Cu") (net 1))
 (segment (start 130.651489 90.836511) (end 128.174511 90.836511) (width 0.25) (layer "F.Cu") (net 1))
 (segment (start 134.379 75.946) (end 134.379 75.601924) (width 0.25) (layer "F.Cu") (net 1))
 (segment (start 134.379 75.601924) (end 133.474045 74.696969) (width 0.25) (layer "F.Cu") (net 1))
 (segment (start 134.379 75.946) (end 134.588 76.155) (width 0.25) (layer "F.Cu") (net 1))
 (segment (start 125.984 79.185) (end 124.19002 79.185) (width 0.25) (layer "F.Cu") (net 1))
 (segment (start 128.553031 74.696969) (end 123.08602 80.16398) (width 0.25) (layer "F.Cu") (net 1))
 (segment (start 128.174511 90.836511) (end 128.016 90.678) (width 0.25) (layer "F.Cu") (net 1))
 (segment (start 131.826 89.662) (end 132.603974 88.884026) (width 0.25) (layer "F.Cu") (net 1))
 (segment (start 132.603974 88.407974) (end 132.188 87.992) (width 0.25) (layer "F.Cu") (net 1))
 (via (at 125.984 85.344) (size 0.8) (drill 0.4) (layers "F.Cu" "B.Cu") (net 1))
 (via (at 128.016 90.678) (size 0.8) (drill 0.4) (layers "F.Cu" "B.Cu") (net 1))
 (via (at 125.984 84.074) (size 0.8) (drill 0.4) (layers "F.Cu" "B.Cu") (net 1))
 (segment (start 128.016 87.376) (end 125.984 85.344) (width 0.25) (layer "B.Cu") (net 1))
 (segment (start 125.984 84.074) (end 125.984 83.18698) (width 0.25) (layer "B.Cu") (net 1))
 (segment (start 125.984 83.18698) (end 123.08602 80.289) (width 0.25) (layer "B.Cu") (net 1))
 (segment (start 125.984 85.344) (end 125.984 84.074) (width 0.25) (layer "B.Cu") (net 1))
 (segment (start 128.016 90.678) (end 128.016 87.376) (width 0.25) (layer "B.Cu") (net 1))
 (segment (start 134.694 90.35) (end 134.856 90.512) (width 0.25) (layer "F.Cu") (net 11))
 (segment (start 134.588 90.244) (end 134.694 90.35) (width 0.25) (layer "F.Cu") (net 11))
 (segment (start 135.681 90.637) (end 135.806 90.512) (width 0.25) (layer "F.Cu") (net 11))
 (segment (start 135.681 92.27) (end 135.681 90.637) (width 0.25) (layer "F.Cu") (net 11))
 (segment (start 134.856 90.512) (end 135.806 90.512) (width 0.25) (layer "F.Cu") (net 11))
 (segment (start 134.588 86.546) (end 134.588 90.244) (width 0.25) (layer "F.Cu") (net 11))
 (segment (start 139.954 88.887) (end 138.081 88.887) (width 0.25) (layer "F.Cu") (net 3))
 (segment (start 138.081 88.887) (end 138.006 88.812) (width 0.25) (layer "F.Cu") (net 3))
 (segment (start 135.388 86.546) (end 135.74 86.546) (width 0.25) (layer "F.Cu") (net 3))
 (segment (start 135.74 86.546) (end 138.006 88.812) (width 0.25) (layer "F.Cu") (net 3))
 (segment (start 124.81902 81.096) (end 123.08602 82.829) (width 0.25) (layer "F.Cu") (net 12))
 (segment (start 128.338 81.096) (end 124.81902 81.096) (width 0.25) (layer "F.Cu") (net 12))
 (segment (start 126.55902 81.896) (end 123.08602 85.369) (width 0.25) (layer "F.Cu") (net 2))
 (segment (start 128.338 81.896) (end 126.55902 81.896) (width 0.25) (layer "F.Cu") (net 2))
 (segment (start 132.538732 82.745268) (end 132.538732 82.86249) (width 0.25) (layer "F.Cu") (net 5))
 (segment (start 135.788 79.496) (end 132.538732 82.745268) (width 0.25) (layer "F.Cu") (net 5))
 (segment (start 132.538732 82.86249) (end 132.247233 83.153989) (width 0.25) (layer "F.Cu") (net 5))
 (segment (start 136.838 79.496) (end 135.788 79.496) (width 0.25) (layer "F.Cu") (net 5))
 (segment (start 132.247233 83.153989) (end 131.588034 83.153989) (width 0.25) (layer "F.Cu") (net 5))
 (via (at 131.588034 83.153989) (size 0.8) (drill 0.4) (layers "F.Cu" "B.Cu") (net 5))
 (segment (start 132.11319 84.234894) (end 131.884489 84.006193) (width 0.25) (layer "B.Cu") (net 5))
 (segment (start 131.884489 83.450444) (end 131.588034 83.153989) (width 0.25) (layer "B.Cu") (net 5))
 (segment (start 133.000511 91.027489) (end 133.000511 89.058511) (width 0.25) (layer "B.Cu") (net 5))
 (segment (start 132.11319 88.17119) (end 132.11319 84.234894) (width 0.25) (layer "B.Cu") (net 5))
 (segment (start 133.000511 89.058511) (end 132.11319 88.17119) (width 0.25) (layer "B.Cu") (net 5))
 (segment (start 131.826 92.202) (end 133.000511 91.027489) (width 0.25) (layer "B.Cu") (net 5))
 (segment (start 131.884489 84.006193) (end 131.884489 83.450444) (width 0.25) (layer "B.Cu") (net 5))
 (segment (start 135.388 79.260282) (end 133.114282 81.534) (width 0.25) (layer "F.Cu") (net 6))
 (segment (start 133.114282 81.534) (end 131.318 81.534) (width 0.25) (layer "F.Cu") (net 6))
 (segment (start 135.388 78.046) (end 135.388 79.260282) (width 0.25) (layer "F.Cu") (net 6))
 (via (at 131.318 81.534) (size 0.8) (drill 0.4) (layers "F.Cu" "B.Cu") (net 6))
 (segment (start 130.460511 91.027489) (end 129.286 92.202) (width 0.25) (layer "B.Cu") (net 6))
 (segment (start 130.460511 89.249489) (end 130.460511 91.027489) (width 0.25) (layer "B.Cu") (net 6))
 (segment (start 131.288363 83.960003) (end 131.288363 88.421637) (width 0.25) (layer "B.Cu") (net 6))
 (segment (start 130.863533 83.535173) (end 131.288363 83.960003) (width 0.25) (layer "B.Cu") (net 6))
 (segment (start 131.287935 81.564065) (end 131.287935 82.429488) (width 0.25) (layer "B.Cu") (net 6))
 (segment (start 131.318 81.534) (end 131.287935 81.564065) (width 0.25) (layer "B.Cu") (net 6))
 (segment (start 131.287935 82.429488) (end 130.863533 82.85389) (width 0.25) (layer "B.Cu") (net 6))
 (segment (start 131.288363 88.421637) (end 130.460511 89.249489) (width 0.25) (layer "B.Cu") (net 6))
 (segment (start 130.863533 82.85389) (end 130.863533 83.535173) (width 0.25) (layer "B.Cu") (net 6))
 (segment (start 135.753359 80.296) (end 132.17087 83.878489) (width 0.25) (layer "F.Cu") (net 7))
 (segment (start 132.17087 83.878489) (end 131.206849 83.878489) (width 0.25) (layer "F.Cu") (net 7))
 (segment (start 130.685375 83.357015) (end 130.139033 83.357015) (width 0.25) (layer "F.Cu") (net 7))
 (segment (start 131.206849 83.878489) (end 130.685375 83.357015) (width 0.25) (layer "F.Cu") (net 7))
 (segment (start 136.838 80.296) (end 135.753359 80.296) (width 0.25) (layer "F.Cu") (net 7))
 (via (at 130.139033 83.357015) (size 0.8) (drill 0.4) (layers "F.Cu" "B.Cu") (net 7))
 (segment (start 129.286 84.210048) (end 130.139033 83.357015) (width 0.25) (layer "B.Cu") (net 7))
 (segment (start 129.286 89.662) (end 129.286 84.210048) (width 0.25) (layer "B.Cu") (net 7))
 (segment (start 125.571489 87.343511) (end 125.571489 91.027489) (width 0.25) (layer "F.Cu") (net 8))
 (segment (start 125.571489 91.027489) (end 126.746 92.202) (width 0.25) (layer "F.Cu") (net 8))
 (segment (start 127.288 82.696) (end 126.78352 83.20048) (width 0.25) (layer "F.Cu") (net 8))
 (segment (start 125.984 86.931) (end 125.571489 87.343511) (width 0.25) (layer "F.Cu") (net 8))
 (segment (start 126.78352 83.20048) (end 126.78352 86.13148) (width 0.25) (layer "F.Cu") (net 8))
 (segment (start 128.338 82.696) (end 127.288 82.696) (width 0.25) (layer "F.Cu") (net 8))
 (segment (start 126.78352 86.13148) (end 125.984 86.931) (width 0.25) (layer "F.Cu") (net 8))
 (segment (start 134.042099 85.269693) (end 134.466501 84.845291) (width 0.25) (layer "F.Cu") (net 9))
 (segment (start 129.788 85.496) (end 130.343126 84.940874) (width 0.25) (layer "F.Cu") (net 9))
 (segment (start 130.343126 84.940874) (end 132.904261 84.940874) (width 0.25) (layer "F.Cu") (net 9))
 (segment (start 133.23308 85.269693) (end 134.042099 85.269693) (width 0.25) (layer "F.Cu") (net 9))
 (segment (start 129.788 86.546) (end 129.788 85.496) (width 0.25) (layer "F.Cu") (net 9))
 (segment (start 134.466501 84.845291) (end 134.466501 84.245093) (width 0.25) (layer "F.Cu") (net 9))
 (segment (start 134.450916 84.229508) (end 134.450916 83.840604) (width 0.25) (layer "F.Cu") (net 9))
 (segment (start 132.904261 84.940874) (end 133.23308 85.269693) (width 0.25) (layer "F.Cu") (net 9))
 (segment (start 134.466501 84.245093) (end 134.450916 84.229508) (width 0.25) (layer "F.Cu") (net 9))
 (via (at 134.450916 83.840604) (size 0.8) (drill 0.4) (layers "F.Cu" "B.Cu") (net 9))
 (segment (start 142.90198 82.829) (end 135.46252 82.829) (width 0.25) (layer "B.Cu") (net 9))
 (segment (start 135.46252 82.829) (end 134.450916 83.840604) (width 0.25) (layer "B.Cu") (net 9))
 (segment (start 133.742 84.545192) (end 133.524808 84.328) (width 0.25) (layer "F.Cu") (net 10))
 (segment (start 130.156 84.328) (end 129.388 85.096) (width 0.25) (layer "F.Cu") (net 10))
 (segment (start 129.388 85.096) (end 128.338 85.096) (width 0.25) (layer "F.Cu") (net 10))
 (segment (start 133.524808 84.328) (end 130.156 84.328) (width 0.25) (layer "F.Cu") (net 10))
 (via (at 133.742 84.545192) (size 0.8) (drill 0.4) (layers "F.Cu" "B.Cu") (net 10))
 (segment (start 134.565808 85.369) (end 133.742 84.545192) (width 0.25) (layer "B.Cu") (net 10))
 (segment (start 142.90198 85.369) (end 134.565808 85.369) (width 0.25) (layer "B.Cu") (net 10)))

